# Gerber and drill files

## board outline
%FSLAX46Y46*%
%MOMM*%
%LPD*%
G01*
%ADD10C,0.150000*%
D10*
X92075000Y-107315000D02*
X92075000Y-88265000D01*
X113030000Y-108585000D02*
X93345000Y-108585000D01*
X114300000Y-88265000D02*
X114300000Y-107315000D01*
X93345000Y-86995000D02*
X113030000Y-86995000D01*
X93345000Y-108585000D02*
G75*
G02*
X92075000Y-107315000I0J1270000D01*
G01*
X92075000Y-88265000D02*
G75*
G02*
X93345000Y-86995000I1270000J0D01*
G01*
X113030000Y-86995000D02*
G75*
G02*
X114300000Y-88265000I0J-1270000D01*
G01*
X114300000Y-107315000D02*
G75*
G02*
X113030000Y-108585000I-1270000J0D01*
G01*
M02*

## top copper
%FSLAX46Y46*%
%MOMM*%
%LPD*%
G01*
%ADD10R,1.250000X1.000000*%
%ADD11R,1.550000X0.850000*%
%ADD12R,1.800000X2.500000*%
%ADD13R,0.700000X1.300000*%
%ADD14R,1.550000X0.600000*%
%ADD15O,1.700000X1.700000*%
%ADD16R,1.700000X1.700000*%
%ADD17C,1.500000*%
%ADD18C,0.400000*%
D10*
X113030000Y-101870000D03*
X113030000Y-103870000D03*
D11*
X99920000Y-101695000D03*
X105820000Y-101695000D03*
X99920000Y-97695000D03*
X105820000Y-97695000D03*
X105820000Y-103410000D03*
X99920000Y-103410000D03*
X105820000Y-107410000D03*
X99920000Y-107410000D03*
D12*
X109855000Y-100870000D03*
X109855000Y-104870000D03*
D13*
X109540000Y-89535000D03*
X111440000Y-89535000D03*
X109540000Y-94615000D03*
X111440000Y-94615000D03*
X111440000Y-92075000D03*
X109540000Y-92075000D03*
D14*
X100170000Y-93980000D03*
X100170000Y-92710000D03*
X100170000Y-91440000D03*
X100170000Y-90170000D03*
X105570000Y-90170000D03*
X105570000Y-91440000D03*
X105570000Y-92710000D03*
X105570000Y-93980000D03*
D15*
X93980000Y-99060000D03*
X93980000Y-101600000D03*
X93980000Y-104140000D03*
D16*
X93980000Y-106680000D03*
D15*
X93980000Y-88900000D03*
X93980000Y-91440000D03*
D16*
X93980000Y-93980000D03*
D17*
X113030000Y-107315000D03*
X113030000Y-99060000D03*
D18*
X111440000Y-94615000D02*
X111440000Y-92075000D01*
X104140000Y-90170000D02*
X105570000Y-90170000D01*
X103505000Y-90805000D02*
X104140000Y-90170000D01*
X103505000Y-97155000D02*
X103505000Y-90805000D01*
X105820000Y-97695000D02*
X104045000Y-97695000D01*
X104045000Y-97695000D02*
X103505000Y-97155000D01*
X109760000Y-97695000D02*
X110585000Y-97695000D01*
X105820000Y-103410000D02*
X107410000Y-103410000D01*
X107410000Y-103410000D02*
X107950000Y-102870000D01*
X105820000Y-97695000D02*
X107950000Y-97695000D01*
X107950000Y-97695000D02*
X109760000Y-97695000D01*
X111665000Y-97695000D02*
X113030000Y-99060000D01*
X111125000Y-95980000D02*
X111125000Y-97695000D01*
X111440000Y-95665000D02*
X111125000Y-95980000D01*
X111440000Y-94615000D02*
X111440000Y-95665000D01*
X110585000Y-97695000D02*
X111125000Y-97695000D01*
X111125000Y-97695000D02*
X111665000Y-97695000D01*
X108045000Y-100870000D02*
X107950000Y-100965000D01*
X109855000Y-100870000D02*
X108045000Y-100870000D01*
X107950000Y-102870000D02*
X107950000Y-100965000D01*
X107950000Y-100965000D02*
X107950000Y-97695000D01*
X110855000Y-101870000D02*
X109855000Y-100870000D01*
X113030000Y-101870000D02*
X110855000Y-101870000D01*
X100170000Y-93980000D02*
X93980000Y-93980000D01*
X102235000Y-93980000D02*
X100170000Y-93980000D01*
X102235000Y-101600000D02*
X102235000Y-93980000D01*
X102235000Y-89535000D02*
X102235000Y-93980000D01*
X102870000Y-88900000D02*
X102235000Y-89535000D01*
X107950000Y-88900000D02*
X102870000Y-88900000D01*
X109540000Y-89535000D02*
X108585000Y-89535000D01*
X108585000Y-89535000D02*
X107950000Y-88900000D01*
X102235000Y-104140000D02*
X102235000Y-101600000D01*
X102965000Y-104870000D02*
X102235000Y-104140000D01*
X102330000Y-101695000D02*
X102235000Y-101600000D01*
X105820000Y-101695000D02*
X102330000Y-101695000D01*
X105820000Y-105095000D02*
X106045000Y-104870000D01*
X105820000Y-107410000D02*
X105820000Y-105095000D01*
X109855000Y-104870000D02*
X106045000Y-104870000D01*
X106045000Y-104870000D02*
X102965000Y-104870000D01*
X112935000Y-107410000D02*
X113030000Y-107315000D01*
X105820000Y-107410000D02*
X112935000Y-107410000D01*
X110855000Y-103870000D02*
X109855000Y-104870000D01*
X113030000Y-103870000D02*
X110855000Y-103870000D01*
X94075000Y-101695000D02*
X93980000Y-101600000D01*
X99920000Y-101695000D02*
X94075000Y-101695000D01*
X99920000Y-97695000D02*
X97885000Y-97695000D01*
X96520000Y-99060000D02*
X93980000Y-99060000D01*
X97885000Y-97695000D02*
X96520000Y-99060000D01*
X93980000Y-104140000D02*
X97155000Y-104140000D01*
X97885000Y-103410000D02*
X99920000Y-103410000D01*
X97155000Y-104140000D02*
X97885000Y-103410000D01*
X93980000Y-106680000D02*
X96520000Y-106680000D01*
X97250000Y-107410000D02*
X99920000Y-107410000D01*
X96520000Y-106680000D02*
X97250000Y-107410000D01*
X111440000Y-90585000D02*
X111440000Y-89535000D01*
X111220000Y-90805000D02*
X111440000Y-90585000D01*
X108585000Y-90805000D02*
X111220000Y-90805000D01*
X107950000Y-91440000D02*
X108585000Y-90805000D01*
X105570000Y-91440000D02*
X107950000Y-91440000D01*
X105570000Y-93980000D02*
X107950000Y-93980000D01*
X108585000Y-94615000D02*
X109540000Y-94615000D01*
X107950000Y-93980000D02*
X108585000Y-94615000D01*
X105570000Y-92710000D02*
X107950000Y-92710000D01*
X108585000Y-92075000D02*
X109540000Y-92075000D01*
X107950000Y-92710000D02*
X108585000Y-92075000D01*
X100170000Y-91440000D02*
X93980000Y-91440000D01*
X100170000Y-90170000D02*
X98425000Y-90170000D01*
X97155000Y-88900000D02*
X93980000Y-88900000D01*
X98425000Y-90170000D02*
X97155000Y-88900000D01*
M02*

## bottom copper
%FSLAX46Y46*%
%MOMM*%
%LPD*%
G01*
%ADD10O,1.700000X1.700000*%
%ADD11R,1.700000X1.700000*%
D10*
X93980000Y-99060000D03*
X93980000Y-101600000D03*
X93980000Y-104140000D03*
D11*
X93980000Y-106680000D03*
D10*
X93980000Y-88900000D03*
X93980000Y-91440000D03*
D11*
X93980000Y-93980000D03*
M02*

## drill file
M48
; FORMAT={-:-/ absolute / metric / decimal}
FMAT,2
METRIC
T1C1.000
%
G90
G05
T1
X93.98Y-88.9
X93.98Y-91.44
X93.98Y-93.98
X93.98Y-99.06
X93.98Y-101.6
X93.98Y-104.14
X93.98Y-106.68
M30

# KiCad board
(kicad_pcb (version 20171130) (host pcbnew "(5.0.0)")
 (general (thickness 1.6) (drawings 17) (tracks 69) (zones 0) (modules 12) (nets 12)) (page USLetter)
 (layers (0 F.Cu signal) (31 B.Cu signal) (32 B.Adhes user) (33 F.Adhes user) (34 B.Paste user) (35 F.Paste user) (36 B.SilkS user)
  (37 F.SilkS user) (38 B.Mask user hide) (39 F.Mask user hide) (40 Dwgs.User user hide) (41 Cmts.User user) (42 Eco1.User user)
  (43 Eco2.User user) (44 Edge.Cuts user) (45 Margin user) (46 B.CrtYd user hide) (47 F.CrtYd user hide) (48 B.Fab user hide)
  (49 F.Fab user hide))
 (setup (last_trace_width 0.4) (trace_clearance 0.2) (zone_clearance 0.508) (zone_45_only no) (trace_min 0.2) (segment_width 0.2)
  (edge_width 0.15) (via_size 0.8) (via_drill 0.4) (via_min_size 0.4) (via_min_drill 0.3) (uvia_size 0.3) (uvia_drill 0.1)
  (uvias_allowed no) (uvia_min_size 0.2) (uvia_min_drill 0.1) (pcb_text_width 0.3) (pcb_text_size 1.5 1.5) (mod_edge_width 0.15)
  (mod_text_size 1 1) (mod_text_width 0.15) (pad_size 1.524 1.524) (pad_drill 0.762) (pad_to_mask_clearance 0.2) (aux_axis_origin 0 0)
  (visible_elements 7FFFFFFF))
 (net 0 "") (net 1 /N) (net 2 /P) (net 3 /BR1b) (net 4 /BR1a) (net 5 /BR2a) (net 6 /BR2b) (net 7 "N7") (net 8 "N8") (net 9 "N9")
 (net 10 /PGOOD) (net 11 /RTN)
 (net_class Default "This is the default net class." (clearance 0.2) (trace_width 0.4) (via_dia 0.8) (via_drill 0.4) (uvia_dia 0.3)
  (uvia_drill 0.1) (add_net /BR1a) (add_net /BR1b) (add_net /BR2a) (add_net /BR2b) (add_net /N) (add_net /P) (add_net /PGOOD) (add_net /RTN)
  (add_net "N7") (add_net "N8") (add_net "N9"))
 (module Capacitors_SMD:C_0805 (layer F.Cu) (at 113.03 102.87 90)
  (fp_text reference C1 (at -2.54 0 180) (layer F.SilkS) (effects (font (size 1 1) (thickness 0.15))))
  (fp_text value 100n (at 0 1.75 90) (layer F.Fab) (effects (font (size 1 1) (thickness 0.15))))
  (pad 2 smd rect (at 1 0 90) (size 1 1.25) (layers F.Cu F.Paste F.Mask) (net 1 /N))
  (pad 1 smd rect (at -1 0 90) (size 1 1.25) (layers F.Cu F.Paste F.Mask) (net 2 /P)))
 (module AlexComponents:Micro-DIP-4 (layer F.Cu) (at 102.87 99.695 90)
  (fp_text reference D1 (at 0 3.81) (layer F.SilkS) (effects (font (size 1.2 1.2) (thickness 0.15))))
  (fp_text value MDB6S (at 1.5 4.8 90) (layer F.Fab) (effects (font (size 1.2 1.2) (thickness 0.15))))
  (pad 4 smd rect (at -2 -2.95 90) (size 0.85 1.55) (layers F.Cu F.Paste F.Mask) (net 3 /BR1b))
  (pad 1 smd rect (at -2 2.95 90) (size 0.85 1.55) (layers F.Cu F.Paste F.Mask) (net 2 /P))
  (pad 3 smd rect (at 2 -2.95 90) (size 0.85 1.55) (layers F.Cu F.Paste F.Mask) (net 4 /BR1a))
  (pad 2 smd rect (at 2 2.95 90) (size 0.85 1.55) (layers F.Cu F.Paste F.Mask) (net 1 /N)))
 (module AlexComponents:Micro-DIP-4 (layer F.Cu) (at 102.87 105.41 90)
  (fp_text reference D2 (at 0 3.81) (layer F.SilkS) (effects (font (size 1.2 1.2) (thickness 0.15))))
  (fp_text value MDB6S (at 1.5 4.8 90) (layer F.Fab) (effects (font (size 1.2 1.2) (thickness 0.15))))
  (pad 2 smd rect (at 2 2.95 90) (size 0.85 1.55) (layers F.Cu F.Paste F.Mask) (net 1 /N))
  (pad 3 smd rect (at 2 -2.95 90) (size 0.85 1.55) (layers F.Cu F.Paste F.Mask) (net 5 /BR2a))
  (pad 1 smd rect (at -2 2.95 90) (size 0.85 1.55) (layers F.Cu F.Paste F.Mask) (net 2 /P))
  (pad 4 smd rect (at -2 -2.95 90) (size 0.85 1.55) (layers F.Cu F.Paste F.Mask) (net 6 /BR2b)))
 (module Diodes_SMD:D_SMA (layer F.Cu) (at 109.855 102.87 90)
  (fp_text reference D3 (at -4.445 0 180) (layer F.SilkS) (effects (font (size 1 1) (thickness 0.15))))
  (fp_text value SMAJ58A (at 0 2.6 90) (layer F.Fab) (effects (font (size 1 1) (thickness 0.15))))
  (pad 2 smd rect (at 2 0 90) (size 2.5 1.8) (layers F.Cu F.Paste F.Mask) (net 1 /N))
  (pad 1 smd rect (at -2 0 90) (size 2.5 1.8) (layers F.Cu F.Paste F.Mask) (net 2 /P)))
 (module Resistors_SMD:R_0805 (layer F.Cu) (at 110.49 89.535 180)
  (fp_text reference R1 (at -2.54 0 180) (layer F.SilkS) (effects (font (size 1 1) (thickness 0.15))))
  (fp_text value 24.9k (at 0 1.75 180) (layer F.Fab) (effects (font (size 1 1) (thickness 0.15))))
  (pad 2 smd rect (at 0.95 0 180) (size 0.7 1.3) (layers F.Cu F.Paste F.Mask) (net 2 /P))
  (pad 1 smd rect (at -0.95 0 180) (size 0.7 1.3) (layers F.Cu F.Paste F.Mask) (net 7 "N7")))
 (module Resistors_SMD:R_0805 (layer F.Cu) (at 110.49 94.615 180)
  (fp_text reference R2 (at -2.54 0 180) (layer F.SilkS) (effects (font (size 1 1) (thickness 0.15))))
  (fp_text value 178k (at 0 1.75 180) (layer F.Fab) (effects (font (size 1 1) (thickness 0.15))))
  (pad 2 smd rect (at 0.95 0 180) (size 0.7 1.3) (layers F.Cu F.Paste F.Mask) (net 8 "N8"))
  (pad 1 smd rect (at -0.95 0 180) (size 0.7 1.3) (layers F.Cu F.Paste F.Mask) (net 1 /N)))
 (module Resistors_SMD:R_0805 (layer F.Cu) (at 110.49 92.075 180)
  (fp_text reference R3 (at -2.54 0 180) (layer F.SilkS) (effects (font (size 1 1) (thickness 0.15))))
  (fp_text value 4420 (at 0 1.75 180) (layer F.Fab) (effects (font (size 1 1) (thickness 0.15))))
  (pad 1 smd rect (at -0.95 0 180) (size 0.7 1.3) (layers F.Cu F.Paste F.Mask) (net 1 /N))
  (pad 2 smd rect (at 0.95 0 180) (size 0.7 1.3) (layers F.Cu F.Paste F.Mask) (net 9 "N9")))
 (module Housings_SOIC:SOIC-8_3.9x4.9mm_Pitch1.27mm (layer F.Cu) (at 102.87 92.075 180)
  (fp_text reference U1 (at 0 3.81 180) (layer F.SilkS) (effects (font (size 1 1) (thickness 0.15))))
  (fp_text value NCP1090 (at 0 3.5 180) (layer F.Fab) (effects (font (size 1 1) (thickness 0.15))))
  (pad 8 smd rect (at 2.7 -1.905 180) (size 1.55 0.6) (layers F.Cu F.Paste F.Mask) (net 2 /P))
  (pad 7 smd rect (at 2.7 -0.635 180) (size 1.55 0.6) (layers F.Cu F.Paste F.Mask))
  (pad 6 smd rect (at 2.7 0.635 180) (size 1.55 0.6) (layers F.Cu F.Paste F.Mask) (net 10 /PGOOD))
  (pad 5 smd rect (at 2.7 1.905 180) (size 1.55 0.6) (layers F.Cu F.Paste F.Mask) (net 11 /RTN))
  (pad 4 smd rect (at -2.7 1.905 180) (size 1.55 0.6) (layers F.Cu F.Paste F.Mask) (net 1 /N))
  (pad 3 smd rect (at -2.7 0.635 180) (size 1.55 0.6) (layers F.Cu F.Paste F.Mask) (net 7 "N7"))
  (pad 2 smd rect (at -2.7 -0.635 180) (size 1.55 0.6) (layers F.Cu F.Paste F.Mask) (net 9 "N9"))
  (pad 1 smd rect (at -2.7 -1.905 180) (size 1.55 0.6) (layers F.Cu F.Paste F.Mask) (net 8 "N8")))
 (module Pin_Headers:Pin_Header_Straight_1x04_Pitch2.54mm (layer B.Cu) (at 93.98 106.68)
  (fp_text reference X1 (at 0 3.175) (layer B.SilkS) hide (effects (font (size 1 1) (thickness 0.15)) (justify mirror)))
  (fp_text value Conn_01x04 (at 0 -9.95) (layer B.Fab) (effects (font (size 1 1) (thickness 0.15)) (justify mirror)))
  (pad 4 thru_hole oval (at 0 -7.62) (size 1.7 1.7) (drill 1) (layers *.Cu *.Mask) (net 4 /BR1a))
  (pad 3 thru_hole oval (at 0 -5.08) (size 1.7 1.7) (drill 1) (layers *.Cu *.Mask) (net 3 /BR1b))
  (pad 2 thru_hole oval (at 0 -2.54) (size 1.7 1.7) (drill 1) (layers *.Cu *.Mask) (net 5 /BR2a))
  (pad 1 thru_hole rect (at 0 0) (size 1.7 1.7) (drill 1) (layers *.Cu *.Mask) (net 6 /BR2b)))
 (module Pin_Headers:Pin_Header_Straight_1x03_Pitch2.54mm (layer B.Cu) (at 93.98 93.98)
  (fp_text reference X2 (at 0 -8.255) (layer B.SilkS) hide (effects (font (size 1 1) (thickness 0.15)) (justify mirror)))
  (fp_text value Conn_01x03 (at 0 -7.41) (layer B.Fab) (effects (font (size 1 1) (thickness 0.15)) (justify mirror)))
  (pad 3 thru_hole oval (at 0 -5.08) (size 1.7 1.7) (drill 1) (layers *.Cu *.Mask) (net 11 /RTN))
  (pad 2 thru_hole oval (at 0 -2.54) (size 1.7 1.7) (drill 1) (layers *.Cu *.Mask) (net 10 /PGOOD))
  (pad 1 thru_hole rect (at 0 0) (size 1.7 1.7) (drill 1) (layers *.Cu *.Mask) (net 2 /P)))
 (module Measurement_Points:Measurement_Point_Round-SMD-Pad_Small (layer F.Cu) (at 113.03 107.315)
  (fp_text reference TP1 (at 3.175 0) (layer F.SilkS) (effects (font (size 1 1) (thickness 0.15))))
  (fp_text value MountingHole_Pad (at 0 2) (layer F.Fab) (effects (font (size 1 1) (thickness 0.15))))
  (pad 1 smd circle (at 0 0) (size 1.5 1.5) (layers F.Cu F.Mask) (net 2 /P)))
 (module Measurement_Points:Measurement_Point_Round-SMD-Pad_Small (layer F.Cu) (at 113.03 99.06)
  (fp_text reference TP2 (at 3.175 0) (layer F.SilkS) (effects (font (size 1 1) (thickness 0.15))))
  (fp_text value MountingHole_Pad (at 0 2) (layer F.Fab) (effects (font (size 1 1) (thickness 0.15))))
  (pad 1 smd circle (at 0 0) (size 1.5 1.5) (layers F.Cu F.Mask) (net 1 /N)))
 (gr_line (start 92.075 107.315) (end 92.075 88.265) (layer Edge.Cuts) (width 0.15))
 (gr_line (start 113.03 108.585) (end 93.345 108.585) (layer Edge.Cuts) (width 0.15))
 (gr_line (start 114.3 88.265) (end 114.3 107.315) (layer Edge.Cuts) (width 0.15))
 (gr_line (start 93.345 86.995) (end 113.03 86.995) (layer Edge.Cuts) (width 0.15))
 (gr_arc (start 93.345 107.315) (end 92.075 107.315) (angle -90) (layer Edge.Cuts) (width 0.15))
 (gr_arc (start 93.345 88.265) (end 93.345 86.995) (angle -90) (layer Edge.Cuts) (width 0.15))
 (gr_arc (start 113.03 88.265) (end 114.3 88.265) (angle -90) (layer Edge.Cuts) (width 0.15))
 (gr_arc (start 113.03 107.315) (end 113.03 108.585) (angle -90) (layer Edge.Cuts) (width 0.15))
 (segment (start 111.44 94.615) (end 111.44 92.075) (width 0.4) (layer F.Cu) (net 1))
 (segment (start 104.14 90.17) (end 105.57 90.17) (width 0.4) (layer F.Cu) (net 1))
 (segment (start 103.505 90.805) (end 104.14 90.17) (width 0.4) (layer F.Cu) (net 1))
 (segment (start 103.505 97.155) (end 103.505 90.805) (width 0.4) (layer F.Cu) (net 1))
 (segment (start 105.82 97.695) (end 104.045 97.695) (width 0.4) (layer F.Cu) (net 1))
 (segment (start 104.045 97.695) (end 103.505 97.155) (width 0.4) (layer F.Cu) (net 1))
 (segment (start 109.76 97.695) (end 110.585 97.695) (width 0.4) (layer F.Cu) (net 1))
 (segment (start 105.82 103.41) (end 107.41 103.41) (width 0.4) (layer F.Cu) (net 1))
 (segment (start 107.41 103.41) (end 107.95 102.87) (width 0.4) (layer F.Cu) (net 1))
 (segment (start 105.82 97.695) (end 107.95 97.695) (width 0.4) (layer F.Cu) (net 1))
 (segment (start 107.95 97.695) (end 109.76 97.695) (width 0.4) (layer F.Cu) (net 1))
 (segment (start 111.665 97.695) (end 113.03 99.06) (width 0.4) (layer F.Cu) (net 1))
 (segment (start 111.125 95.98) (end 111.125 97.695) (width 0.4) (layer F.Cu) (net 1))
 (segment (start 111.44 95.665) (end 111.125 95.98) (width 0.4) (layer F.Cu) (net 1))
 (segment (start 111.44 94.615) (end 111.44 95.665) (width 0.4) (layer F.Cu) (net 1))
 (segment (start 110.585 97.695) (end 111.125 97.695) (width 0.4) (layer F.Cu) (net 1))
 (segment (start 111.125 97.695) (end 111.665 97.695) (width 0.4) (layer F.Cu) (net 1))
 (segment (start 108.045 100.87) (end 107.95 100.965) (width 0.4) (layer F.Cu) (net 1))
 (segment (start 109.855 100.87) (end 108.045 100.87) (width 0.4) (layer F.Cu) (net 1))
 (segment (start 107.95 102.87) (end 107.95 100.965) (width 0.4) (layer F.Cu) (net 1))
 (segment (start 107.95 100.965) (end 107.95 97.695) (width 0.4) (layer F.Cu) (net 1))
 (segment (start 110.855 101.87) (end 109.855 100.87) (width 0.4) (layer F.Cu) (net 1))
 (segment (start 113.03 101.87) (end 110.855 101.87) (width 0.4) (layer F.Cu) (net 1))
 (segment (start 100.17 93.98) (end 93.98 93.98) (width 0.4) (layer F.Cu) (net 2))
 (segment (start 102.235 93.98) (end 100.17 93.98) (width 0.4) (layer F.Cu) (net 2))
 (segment (start 102.235 101.6) (end 102.235 93.98) (width 0.4) (layer F.Cu) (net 2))
 (segment (start 102.235 89.535) (end 102.235 93.98) (width 0.4) (layer F.Cu) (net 2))
 (segment (start 102.87 88.9) (end 102.235 89.535) (width 0.4) (layer F.Cu) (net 2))
 (segment (start 107.95 88.9) (end 102.87 88.9) (width 0.4) (layer F.Cu) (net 2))
 (segment (start 109.54 89.535) (end 108.585 89.535) (width 0.4) (layer F.Cu) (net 2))
 (segment (start 108.585 89.535) (end 107.95 88.9) (width 0.4) (layer F.Cu) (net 2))
 (segment (start 102.235 104.14) (end 102.235 101.6) (width 0.4) (layer F.Cu) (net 2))
 (segment (start 102.965 104.87) (end 102.235 104.14) (width 0.4) (layer F.Cu) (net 2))
 (segment (start 102.33 101.695) (end 102.235 101.6) (width 0.4) (layer F.Cu) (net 2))
 (segment (start 105.82 101.695) (end 102.33 101.695) (width 0.4) (layer F.Cu) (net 2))
 (segment (start 105.82 105.095) (end 106.045 104.87) (width 0.4) (layer F.Cu) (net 2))
 (segment (start 105.82 107.41) (end 105.82 105.095) (width 0.4) (layer F.Cu) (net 2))
 (segment (start 109.855 104.87) (end 106.045 104.87) (width 0.4) (layer F.Cu) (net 2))
 (segment (start 106.045 104.87) (end 102.965 104.87) (width 0.4) (layer F.Cu) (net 2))
 (segment (start 112.935 107.41) (end 113.03 107.315) (width 0.4) (layer F.Cu) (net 2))
 (segment (start 105.82 107.41) (end 112.935 107.41) (width 0.4) (layer F.Cu) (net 2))
 (segment (start 110.855 103.87) (end 109.855 104.87) (width 0.4) (layer F.Cu) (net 2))
 (segment (start 113.03 103.87) (end 110.855 103.87) (width 0.4) (layer F.Cu) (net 2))
 (segment (start 94.075 101.695) (end 93.98 101.6) (width 0.4) (layer F.Cu) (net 3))
 (segment (start 99.92 101.695) (end 94.075 101.695) (width 0.4) (layer F.Cu) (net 3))
 (segment (start 99.92 97.695) (end 97.885 97.695) (width 0.4) (layer F.Cu) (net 4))
 (segment (start 96.52 99.06) (end 93.98 99.06) (width 0.4) (layer F.Cu) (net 4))
 (segment (start 97.885 97.695) (end 96.52 99.06) (width 0.4) (layer F.Cu) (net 4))
 (segment (start 93.98 104.14) (end 97.155 104.14) (width 0.4) (layer F.Cu) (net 5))
 (segment (start 97.885 103.41) (end 99.92 103.41) (width 0.4) (layer F.Cu) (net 5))
 (segment (start 97.155 104.14) (end 97.885 103.41) (width 0.4) (layer F.Cu) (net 5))
 (segment (start 93.98 106.68) (end 96.52 106.68) (width 0.4) (layer F.Cu) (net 6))
 (segment (start 97.25 107.41) (end 99.92 107.41) (width 0.4) (layer F.Cu) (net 6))
 (segment (start 96.52 106.68) (end 97.25 107.41) (width 0.4) (layer F.Cu) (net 6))
 (segment (start 111.44 90.585) (end 111.44 89.535) (width 0.4) (layer F.Cu) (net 7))
 (segment (start 111.22 90.805) (end 111.44 90.585) (width 0.4) (layer F.Cu) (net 7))
 (segment (start 108.585 90.805) (end 111.22 90.805) (width 0.4) (layer F.Cu) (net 7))
 (segment (start 107.95 91.44) (end 108.585 90.805) (width 0.4) (layer F.Cu) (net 7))
 (segment (start 105.57 91.44) (end 107.95 91.44) (width 0.4) (layer F.Cu) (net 7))
 (segment (start 105.57 93.98) (end 107.95 93.98) (width 0.4) (layer F.Cu) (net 8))
 (segment (start 108.585 94.615) (end 109.54 94.615) (width 0.4) (layer F.Cu) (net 8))
 (segment (start 107.95 93.98) (end 108.585 94.615) (width 0.4) (layer F.Cu) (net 8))
 (segment (start 105.57 92.71) (end 107.95 92.71) (width 0.4) (layer F.Cu) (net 9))
 (segment (start 108.585 92.075) (end 109.54 92.075) (width 0.4) (layer F.Cu) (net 9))
 (segment (start 107.95 92.71) (end 108.585 92.075) (width 0.4) (layer F.Cu) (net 9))
 (segment (start 100.17 91.44) (end 93.98 91.44) (width 0.4) (layer F.Cu) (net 10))
 (segment (start 100.17 90.17) (end 98.425 90.17) (width 0.4) (layer F.Cu) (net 11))
 (segment (start 97.155 88.9) (end 93.98 88.9) (width 0.4) (layer F.Cu) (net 11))
 (segment (start 98.425 90.17) (end 97.155 88.9) (width 0.4) (layer F.Cu) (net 11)))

